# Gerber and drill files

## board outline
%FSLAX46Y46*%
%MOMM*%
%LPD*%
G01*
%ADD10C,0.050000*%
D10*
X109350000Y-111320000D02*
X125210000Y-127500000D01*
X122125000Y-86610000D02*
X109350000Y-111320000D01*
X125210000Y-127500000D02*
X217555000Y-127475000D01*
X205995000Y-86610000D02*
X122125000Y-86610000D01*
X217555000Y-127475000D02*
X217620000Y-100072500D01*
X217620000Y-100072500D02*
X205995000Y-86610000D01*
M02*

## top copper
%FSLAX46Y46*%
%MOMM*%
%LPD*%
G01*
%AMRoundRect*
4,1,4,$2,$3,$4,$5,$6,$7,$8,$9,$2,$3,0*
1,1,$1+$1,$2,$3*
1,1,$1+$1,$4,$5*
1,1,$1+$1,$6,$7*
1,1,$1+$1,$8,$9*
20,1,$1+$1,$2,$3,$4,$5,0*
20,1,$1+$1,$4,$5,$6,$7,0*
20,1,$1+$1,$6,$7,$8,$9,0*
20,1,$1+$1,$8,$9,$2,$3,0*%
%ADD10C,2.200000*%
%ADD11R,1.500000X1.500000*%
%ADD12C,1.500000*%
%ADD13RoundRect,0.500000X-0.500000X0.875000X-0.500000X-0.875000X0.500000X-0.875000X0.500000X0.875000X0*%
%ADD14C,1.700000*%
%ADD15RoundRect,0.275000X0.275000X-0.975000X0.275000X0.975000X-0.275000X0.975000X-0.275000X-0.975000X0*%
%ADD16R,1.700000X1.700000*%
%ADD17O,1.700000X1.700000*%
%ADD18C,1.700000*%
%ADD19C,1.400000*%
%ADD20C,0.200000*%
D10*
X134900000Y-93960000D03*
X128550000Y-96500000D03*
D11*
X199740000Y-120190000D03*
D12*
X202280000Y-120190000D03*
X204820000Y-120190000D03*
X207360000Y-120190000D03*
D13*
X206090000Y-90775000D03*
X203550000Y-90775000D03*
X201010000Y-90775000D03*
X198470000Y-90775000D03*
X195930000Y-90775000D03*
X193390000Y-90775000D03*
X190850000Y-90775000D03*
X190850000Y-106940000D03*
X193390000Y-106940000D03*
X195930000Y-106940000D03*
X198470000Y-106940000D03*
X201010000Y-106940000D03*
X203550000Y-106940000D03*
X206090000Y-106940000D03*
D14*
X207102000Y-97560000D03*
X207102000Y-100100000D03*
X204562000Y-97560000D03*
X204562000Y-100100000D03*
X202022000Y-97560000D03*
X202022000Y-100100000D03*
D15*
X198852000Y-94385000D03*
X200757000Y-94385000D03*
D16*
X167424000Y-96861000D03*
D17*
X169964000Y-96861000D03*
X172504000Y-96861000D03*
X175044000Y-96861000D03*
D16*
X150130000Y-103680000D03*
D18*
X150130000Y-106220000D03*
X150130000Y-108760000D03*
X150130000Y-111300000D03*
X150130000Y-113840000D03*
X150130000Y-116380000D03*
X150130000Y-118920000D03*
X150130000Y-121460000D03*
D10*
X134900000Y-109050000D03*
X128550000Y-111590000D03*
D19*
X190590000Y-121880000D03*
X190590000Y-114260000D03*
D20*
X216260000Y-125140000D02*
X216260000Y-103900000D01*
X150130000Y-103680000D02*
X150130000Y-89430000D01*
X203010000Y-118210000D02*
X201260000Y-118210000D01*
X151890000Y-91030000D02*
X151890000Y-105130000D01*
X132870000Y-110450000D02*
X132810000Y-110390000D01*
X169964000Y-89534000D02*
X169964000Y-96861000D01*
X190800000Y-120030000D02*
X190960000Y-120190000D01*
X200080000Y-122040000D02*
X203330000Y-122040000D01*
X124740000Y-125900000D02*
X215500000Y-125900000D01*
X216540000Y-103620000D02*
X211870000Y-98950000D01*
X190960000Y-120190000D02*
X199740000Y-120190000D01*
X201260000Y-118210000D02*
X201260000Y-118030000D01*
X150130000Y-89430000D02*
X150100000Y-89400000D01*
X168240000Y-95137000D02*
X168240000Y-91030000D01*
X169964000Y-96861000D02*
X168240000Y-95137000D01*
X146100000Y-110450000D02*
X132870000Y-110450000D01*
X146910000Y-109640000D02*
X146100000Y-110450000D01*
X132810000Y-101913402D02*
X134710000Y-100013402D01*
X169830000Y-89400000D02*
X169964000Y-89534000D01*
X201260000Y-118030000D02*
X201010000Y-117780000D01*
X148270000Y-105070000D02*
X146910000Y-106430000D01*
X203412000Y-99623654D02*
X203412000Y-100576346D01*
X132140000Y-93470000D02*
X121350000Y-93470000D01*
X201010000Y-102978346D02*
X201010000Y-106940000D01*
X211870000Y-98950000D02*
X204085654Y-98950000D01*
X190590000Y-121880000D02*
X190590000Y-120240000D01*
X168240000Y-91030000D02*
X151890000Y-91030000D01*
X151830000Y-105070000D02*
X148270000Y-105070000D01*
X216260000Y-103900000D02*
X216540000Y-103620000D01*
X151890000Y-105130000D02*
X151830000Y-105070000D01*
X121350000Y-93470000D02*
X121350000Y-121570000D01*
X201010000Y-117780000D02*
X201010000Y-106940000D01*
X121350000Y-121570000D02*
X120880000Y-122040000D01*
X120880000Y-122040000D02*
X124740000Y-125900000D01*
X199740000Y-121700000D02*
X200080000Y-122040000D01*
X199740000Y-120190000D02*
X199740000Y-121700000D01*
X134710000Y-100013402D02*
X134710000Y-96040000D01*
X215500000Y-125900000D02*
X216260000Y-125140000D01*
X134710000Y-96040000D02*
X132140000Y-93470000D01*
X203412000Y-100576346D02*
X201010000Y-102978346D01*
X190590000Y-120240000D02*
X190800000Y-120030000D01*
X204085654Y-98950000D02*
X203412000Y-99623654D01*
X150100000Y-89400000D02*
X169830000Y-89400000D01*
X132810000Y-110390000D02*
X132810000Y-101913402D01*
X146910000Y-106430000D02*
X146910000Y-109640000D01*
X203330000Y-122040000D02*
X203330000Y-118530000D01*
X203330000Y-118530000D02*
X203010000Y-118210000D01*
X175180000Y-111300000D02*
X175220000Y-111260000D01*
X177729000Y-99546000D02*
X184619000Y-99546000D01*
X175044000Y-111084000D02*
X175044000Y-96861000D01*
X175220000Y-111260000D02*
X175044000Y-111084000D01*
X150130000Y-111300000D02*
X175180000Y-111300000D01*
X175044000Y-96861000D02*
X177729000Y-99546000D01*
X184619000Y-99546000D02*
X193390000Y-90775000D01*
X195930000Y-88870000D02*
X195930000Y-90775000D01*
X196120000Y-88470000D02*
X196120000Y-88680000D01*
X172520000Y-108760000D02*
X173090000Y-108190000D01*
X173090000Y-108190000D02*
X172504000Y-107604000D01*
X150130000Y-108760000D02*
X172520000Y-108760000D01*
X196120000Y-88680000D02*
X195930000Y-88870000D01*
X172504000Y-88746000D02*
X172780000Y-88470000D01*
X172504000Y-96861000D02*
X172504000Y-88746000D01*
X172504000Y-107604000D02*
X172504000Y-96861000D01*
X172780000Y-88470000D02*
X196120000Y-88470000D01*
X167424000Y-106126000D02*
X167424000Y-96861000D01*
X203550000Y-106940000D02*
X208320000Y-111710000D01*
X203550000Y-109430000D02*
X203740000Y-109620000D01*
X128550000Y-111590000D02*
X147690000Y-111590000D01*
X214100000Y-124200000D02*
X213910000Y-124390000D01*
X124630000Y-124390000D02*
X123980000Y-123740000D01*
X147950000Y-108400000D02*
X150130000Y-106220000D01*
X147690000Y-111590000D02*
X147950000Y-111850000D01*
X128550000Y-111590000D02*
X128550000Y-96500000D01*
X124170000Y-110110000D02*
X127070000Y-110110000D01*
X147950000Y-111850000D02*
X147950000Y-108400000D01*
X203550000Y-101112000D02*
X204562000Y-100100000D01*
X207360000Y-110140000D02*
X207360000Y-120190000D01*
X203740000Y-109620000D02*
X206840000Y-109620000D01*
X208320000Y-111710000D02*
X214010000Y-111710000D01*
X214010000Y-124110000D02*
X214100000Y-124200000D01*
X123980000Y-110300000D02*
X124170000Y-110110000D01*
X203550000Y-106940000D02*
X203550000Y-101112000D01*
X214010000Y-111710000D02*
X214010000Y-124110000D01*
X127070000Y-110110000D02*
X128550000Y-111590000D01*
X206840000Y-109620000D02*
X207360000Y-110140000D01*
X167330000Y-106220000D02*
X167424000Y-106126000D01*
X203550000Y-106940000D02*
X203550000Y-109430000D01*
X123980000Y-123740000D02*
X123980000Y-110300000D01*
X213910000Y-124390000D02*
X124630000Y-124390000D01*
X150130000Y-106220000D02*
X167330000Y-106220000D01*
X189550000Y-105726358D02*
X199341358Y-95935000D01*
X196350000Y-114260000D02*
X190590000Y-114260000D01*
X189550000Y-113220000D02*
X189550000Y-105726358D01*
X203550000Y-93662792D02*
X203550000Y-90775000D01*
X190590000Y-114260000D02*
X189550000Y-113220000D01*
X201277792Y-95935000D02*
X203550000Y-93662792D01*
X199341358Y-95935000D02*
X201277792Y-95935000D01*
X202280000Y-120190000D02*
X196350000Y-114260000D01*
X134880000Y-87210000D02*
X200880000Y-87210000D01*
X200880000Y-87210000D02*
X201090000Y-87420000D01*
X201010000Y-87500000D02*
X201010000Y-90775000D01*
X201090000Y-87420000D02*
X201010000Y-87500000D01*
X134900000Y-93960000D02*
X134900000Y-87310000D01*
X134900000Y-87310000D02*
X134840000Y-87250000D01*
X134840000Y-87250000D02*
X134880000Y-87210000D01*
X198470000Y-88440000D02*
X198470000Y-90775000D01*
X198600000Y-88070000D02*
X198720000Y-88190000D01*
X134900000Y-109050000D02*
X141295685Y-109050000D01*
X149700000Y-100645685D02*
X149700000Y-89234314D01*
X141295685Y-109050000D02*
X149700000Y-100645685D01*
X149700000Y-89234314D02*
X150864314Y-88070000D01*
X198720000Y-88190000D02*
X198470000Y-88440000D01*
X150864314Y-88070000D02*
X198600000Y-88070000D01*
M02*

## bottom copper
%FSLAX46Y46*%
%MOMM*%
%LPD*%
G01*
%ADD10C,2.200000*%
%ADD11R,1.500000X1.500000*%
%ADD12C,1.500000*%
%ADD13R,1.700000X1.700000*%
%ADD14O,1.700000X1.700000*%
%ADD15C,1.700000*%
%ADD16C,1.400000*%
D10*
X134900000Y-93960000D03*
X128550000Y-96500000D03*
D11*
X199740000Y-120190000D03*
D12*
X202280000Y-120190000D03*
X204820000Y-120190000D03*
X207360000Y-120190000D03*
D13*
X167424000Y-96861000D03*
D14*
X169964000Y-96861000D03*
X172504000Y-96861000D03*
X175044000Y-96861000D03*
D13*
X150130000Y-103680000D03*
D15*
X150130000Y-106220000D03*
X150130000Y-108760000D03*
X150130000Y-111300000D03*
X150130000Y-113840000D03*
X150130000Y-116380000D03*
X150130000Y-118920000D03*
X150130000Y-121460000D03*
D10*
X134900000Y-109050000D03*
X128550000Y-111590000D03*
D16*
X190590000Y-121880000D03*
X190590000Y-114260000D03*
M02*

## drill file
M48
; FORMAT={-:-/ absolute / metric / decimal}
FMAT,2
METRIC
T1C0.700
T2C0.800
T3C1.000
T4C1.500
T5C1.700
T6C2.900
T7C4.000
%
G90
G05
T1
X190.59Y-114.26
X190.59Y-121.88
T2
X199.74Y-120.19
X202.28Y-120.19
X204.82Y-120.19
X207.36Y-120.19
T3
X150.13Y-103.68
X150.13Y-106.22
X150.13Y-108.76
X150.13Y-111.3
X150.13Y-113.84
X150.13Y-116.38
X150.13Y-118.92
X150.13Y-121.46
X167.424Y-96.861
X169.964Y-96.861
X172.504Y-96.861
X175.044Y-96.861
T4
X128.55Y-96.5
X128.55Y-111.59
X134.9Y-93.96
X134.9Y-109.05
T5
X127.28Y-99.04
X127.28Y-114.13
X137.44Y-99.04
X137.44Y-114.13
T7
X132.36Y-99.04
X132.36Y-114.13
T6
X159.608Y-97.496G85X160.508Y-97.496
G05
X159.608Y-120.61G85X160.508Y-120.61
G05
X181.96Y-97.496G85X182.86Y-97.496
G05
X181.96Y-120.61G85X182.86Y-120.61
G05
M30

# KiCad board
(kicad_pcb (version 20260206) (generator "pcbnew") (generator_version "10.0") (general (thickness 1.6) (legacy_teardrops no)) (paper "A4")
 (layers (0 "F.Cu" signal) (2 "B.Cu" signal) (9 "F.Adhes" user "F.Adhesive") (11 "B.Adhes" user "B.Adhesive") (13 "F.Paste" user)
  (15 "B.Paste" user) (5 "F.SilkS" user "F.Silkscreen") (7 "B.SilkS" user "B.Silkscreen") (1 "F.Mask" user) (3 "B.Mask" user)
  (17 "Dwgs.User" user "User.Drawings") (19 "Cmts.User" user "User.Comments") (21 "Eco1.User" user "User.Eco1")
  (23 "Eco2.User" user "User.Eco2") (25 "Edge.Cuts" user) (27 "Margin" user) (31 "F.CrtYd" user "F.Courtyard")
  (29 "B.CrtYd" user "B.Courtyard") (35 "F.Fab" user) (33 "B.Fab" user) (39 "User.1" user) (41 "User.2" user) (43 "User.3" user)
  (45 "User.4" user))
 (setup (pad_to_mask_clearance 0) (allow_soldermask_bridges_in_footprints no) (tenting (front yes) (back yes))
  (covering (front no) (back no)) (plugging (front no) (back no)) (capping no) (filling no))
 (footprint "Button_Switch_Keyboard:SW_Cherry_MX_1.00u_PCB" (layer "F.Cu") (at 134.9 93.96)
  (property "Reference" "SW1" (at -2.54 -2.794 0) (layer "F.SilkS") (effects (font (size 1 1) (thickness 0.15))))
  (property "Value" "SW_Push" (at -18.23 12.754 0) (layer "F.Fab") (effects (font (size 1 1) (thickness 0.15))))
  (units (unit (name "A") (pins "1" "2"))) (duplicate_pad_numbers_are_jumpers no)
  (pad "" np_thru_hole circle (at -7.62 5.08) (size 1.7 1.7) (drill 1.7) (layers "*.Cu" "*.Mask"))
  (pad "" np_thru_hole circle (at -2.54 5.08) (size 4 4) (drill 4) (layers "*.Cu" "*.Mask"))
  (pad "" np_thru_hole circle (at 2.54 5.08) (size 1.7 1.7) (drill 1.7) (layers "*.Cu" "*.Mask"))
  (pad "1" thru_hole circle (at 0 0) (size 2.2 2.2) (drill 1.5) (layers "*.Cu" "*.Mask") (remove_unused_layers no) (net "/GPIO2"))
  (pad "2" thru_hole circle (at -6.35 2.54) (size 2.2 2.2) (drill 1.5) (layers "*.Cu" "*.Mask") (remove_unused_layers no) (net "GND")))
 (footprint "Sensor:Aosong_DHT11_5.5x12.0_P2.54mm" (layer "F.Cu") (at 199.74 120.19 90)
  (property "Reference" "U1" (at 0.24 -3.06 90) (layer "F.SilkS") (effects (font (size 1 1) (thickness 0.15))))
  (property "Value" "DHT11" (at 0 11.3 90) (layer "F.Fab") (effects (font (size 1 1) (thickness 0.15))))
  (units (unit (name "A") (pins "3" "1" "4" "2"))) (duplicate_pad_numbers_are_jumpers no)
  (pad "1" thru_hole rect (at 0 0 90) (size 1.5 1.5) (drill 0.8) (layers "*.Cu" "*.Mask") (remove_unused_layers no) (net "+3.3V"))
  (pad "2" thru_hole circle (at 0 2.54 90) (size 1.5 1.5) (drill 0.8) (layers "*.Cu" "*.Mask") (remove_unused_layers no) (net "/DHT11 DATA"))
  (pad "3" thru_hole circle (at 0 5.08 90) (size 1.5 1.5) (drill 0.8) (layers "*.Cu" "*.Mask") (remove_unused_layers no)
   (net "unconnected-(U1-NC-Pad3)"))
  (pad "4" thru_hole circle (at 0 7.62 90) (size 1.5 1.5) (drill 0.8) (layers "*.Cu" "*.Mask") (remove_unused_layers no) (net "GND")))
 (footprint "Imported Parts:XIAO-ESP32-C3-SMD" (layer "F.Cu") (at 187.97 89.94 -90)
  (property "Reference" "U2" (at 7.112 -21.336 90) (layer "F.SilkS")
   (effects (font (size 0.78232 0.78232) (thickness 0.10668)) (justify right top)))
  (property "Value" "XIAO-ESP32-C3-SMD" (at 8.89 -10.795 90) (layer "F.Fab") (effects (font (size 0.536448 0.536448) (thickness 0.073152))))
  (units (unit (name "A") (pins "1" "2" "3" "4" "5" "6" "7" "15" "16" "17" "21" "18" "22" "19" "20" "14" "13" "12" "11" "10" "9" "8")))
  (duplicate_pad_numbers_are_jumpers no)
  (pad "1" smd roundrect (at 0.835 -18.12 270) (size 2.75 2) (layers "F.Cu" "F.Mask" "F.Paste") (roundrect_rratio 0.25)
   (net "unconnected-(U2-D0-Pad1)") (solder_mask_margin 0.0508) (thermal_bridge_angle 45))
  (pad "2" smd roundrect (at 0.835 -15.58 270) (size 2.75 2) (layers "F.Cu" "F.Mask" "F.Paste") (roundrect_rratio 0.25) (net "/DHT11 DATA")
   (solder_mask_margin 0.0508) (thermal_bridge_angle 45))
  (pad "3" smd roundrect (at 0.835 -13.04 270) (size 2.75 2) (layers "F.Cu" "F.Mask" "F.Paste") (roundrect_rratio 0.25) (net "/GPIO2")
   (solder_mask_margin 0.0508) (thermal_bridge_angle 45))
  (pad "4" smd roundrect (at 0.835 -10.5 270) (size 2.75 2) (layers "F.Cu" "F.Mask" "F.Paste") (roundrect_rratio 0.25) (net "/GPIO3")
   (solder_mask_margin 0.0508) (thermal_bridge_angle 45))
  (pad "5" smd roundrect (at 0.835 -7.96 270) (size 2.75 2) (layers "F.Cu" "F.Mask" "F.Paste") (roundrect_rratio 0.25) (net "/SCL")
   (solder_mask_margin 0.0508) (thermal_bridge_angle 45))
  (pad "6" smd roundrect (at 0.835 -5.42 270) (size 2.75 2) (layers "F.Cu" "F.Mask" "F.Paste") (roundrect_rratio 0.25) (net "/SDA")
   (solder_mask_margin 0.0508) (thermal_bridge_angle 45))
  (pad "7" smd roundrect (at 0.835 -2.88 270) (size 2.75 2) (layers "F.Cu" "F.Mask" "F.Paste") (roundrect_rratio 0.25)
   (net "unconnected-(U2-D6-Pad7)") (solder_mask_margin 0.0508) (thermal_bridge_angle 45))
  (pad "8" smd roundrect (at 17 -2.88 270) (size 2.75 2) (layers "F.Cu" "F.Mask" "F.Paste") (roundrect_rratio 0.25)
   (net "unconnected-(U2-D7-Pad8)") (solder_mask_margin 0.0508) (thermal_bridge_angle 45))
  (pad "9" smd roundrect (at 17 -5.42 270) (size 2.75 2) (layers "F.Cu" "F.Mask" "F.Paste") (roundrect_rratio 0.25)
   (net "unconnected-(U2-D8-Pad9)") (solder_mask_margin 0.0508) (thermal_bridge_angle 45))
  (pad "10" smd roundrect (at 17 -7.96 270) (size 2.75 2) (layers "F.Cu" "F.Mask" "F.Paste") (roundrect_rratio 0.25)
   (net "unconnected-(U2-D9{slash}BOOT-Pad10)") (solder_mask_margin 0.0508) (thermal_bridge_angle 45))
  (pad "11" smd roundrect (at 17 -10.5 270) (size 2.75 2) (layers "F.Cu" "F.Mask" "F.Paste") (roundrect_rratio 0.25)
   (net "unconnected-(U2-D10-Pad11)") (solder_mask_margin 0.0508) (thermal_bridge_angle 45))
  (pad "12" smd roundrect (at 17 -13.04 270) (size 2.75 2) (layers "F.Cu" "F.Mask" "F.Paste") (roundrect_rratio 0.25) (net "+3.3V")
   (solder_mask_margin 0.0508) (thermal_bridge_angle 45))
  (pad "13" smd roundrect (at 17 -15.58 270) (size 2.75 2) (layers "F.Cu" "F.Mask" "F.Paste") (roundrect_rratio 0.25) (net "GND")
   (solder_mask_margin 0.0508) (thermal_bridge_angle 45))
  (pad "14" smd roundrect (at 17 -18.12 270) (size 2.75 2) (layers "F.Cu" "F.Mask" "F.Paste") (roundrect_rratio 0.25) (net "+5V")
   (solder_mask_margin 0.0508) (thermal_bridge_angle 45))
  (pad "15" smd circle (at 7.62 -19.132 270) (size 1.7 1.7) (layers "F.Cu" "F.Mask" "F.Paste") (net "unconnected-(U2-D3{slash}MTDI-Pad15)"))
  (pad "16" smd circle (at 10.16 -19.132 270) (size 1.7 1.7) (layers "F.Cu" "F.Mask" "F.Paste") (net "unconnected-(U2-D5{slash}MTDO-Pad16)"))
  (pad "17" smd circle (at 7.62 -16.592 270) (size 1.7 1.7) (layers "F.Cu" "F.Mask" "F.Paste") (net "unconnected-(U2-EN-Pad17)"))
  (pad "18" smd circle (at 10.16 -16.592 270) (size 1.7 1.7) (layers "F.Cu" "F.Mask" "F.Paste") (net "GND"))
  (pad "19" smd circle (at 7.62 -14.052 270) (size 1.7 1.7) (layers "F.Cu" "F.Mask" "F.Paste") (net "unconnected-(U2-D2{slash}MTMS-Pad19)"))
  (pad "20" smd circle (at 10.16 -14.052 270) (size 1.7 1.7) (layers "F.Cu" "F.Mask" "F.Paste") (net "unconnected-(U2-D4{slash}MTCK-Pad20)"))
  (pad "21" smd roundrect (at 4.445 -10.882 90) (size 2.5 1.1) (layers "F.Cu" "F.Mask" "F.Paste") (roundrect_rratio 0.25)
   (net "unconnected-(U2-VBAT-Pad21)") (thermal_bridge_angle 45))
  (pad "22" smd roundrect (at 4.445 -12.787 90) (size 2.5 1.1) (layers "F.Cu" "F.Mask" "F.Paste") (roundrect_rratio 0.25)
   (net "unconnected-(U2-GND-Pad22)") (thermal_bridge_angle 45)))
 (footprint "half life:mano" (layer "F.Cu") (at 180.8 111.37)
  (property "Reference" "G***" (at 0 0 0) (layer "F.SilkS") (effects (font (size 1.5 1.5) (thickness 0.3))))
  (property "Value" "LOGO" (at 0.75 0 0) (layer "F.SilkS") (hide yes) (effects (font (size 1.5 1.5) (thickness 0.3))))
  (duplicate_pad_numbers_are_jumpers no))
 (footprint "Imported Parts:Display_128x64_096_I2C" (layer "F.Cu") (at 171.234 96.861)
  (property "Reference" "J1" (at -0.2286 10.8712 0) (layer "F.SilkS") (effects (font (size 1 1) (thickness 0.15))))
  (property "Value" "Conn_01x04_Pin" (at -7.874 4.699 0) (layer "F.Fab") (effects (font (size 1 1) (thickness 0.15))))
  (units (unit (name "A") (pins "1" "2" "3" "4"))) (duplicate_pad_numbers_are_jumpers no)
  (pad "" np_thru_hole oval (at -11.176 0.635) (size 3.8 2.9) (drill oval 3.8 2.9) (layers "*.Cu" "*.Mask"))
  (pad "" np_thru_hole oval (at -11.176 23.749) (size 3.8 2.9) (drill oval 3.8 2.9) (layers "*.Cu" "*.Mask"))
  (pad "" np_thru_hole oval (at 11.176 0.635) (size 3.8 2.9) (drill oval 3.8 2.9) (layers "*.Cu" "*.Mask"))
  (pad "" np_thru_hole oval (at 11.176 23.749) (size 3.8 2.9) (drill oval 3.8 2.9) (layers "*.Cu" "*.Mask"))
  (pad "1" thru_hole rect (at -3.81 0 90) (size 1.7 1.7) (drill 1) (layers "*.Cu" "*.Mask") (remove_unused_layers no) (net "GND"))
  (pad "2" thru_hole oval (at -1.27 0 90) (size 1.7 1.7) (drill 1) (layers "*.Cu" "*.Mask") (remove_unused_layers no) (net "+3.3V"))
  (pad "3" thru_hole oval (at 1.27 0 90) (size 1.7 1.7) (drill 1) (layers "*.Cu" "*.Mask") (remove_unused_layers no) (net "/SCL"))
  (pad "4" thru_hole oval (at 3.81 0 90) (size 1.7 1.7) (drill 1) (layers "*.Cu" "*.Mask") (remove_unused_layers no) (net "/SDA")))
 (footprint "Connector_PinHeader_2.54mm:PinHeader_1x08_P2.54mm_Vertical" (layer "F.Cu") (at 150.13 103.68)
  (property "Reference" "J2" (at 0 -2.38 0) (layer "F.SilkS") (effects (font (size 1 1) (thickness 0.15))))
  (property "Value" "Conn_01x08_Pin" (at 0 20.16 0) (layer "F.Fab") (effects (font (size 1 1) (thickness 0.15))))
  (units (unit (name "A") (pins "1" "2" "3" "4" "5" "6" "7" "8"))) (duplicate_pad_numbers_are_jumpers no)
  (pad "1" thru_hole rect (at 0 0) (size 1.7 1.7) (drill 1) (layers "*.Cu" "*.Mask") (remove_unused_layers no) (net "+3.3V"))
  (pad "2" thru_hole circle (at 0 2.54) (size 1.7 1.7) (drill 1) (layers "*.Cu" "*.Mask") (remove_unused_layers no) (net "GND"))
  (pad "3" thru_hole circle (at 0 5.08) (size 1.7 1.7) (drill 1) (layers "*.Cu" "*.Mask") (remove_unused_layers no) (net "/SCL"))
  (pad "4" thru_hole circle (at 0 7.62) (size 1.7 1.7) (drill 1) (layers "*.Cu" "*.Mask") (remove_unused_layers no) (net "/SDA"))
  (pad "5" thru_hole circle (at 0 10.16) (size 1.7 1.7) (drill 1) (layers "*.Cu" "*.Mask") (remove_unused_layers no)
   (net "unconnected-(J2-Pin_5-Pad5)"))
  (pad "6" thru_hole circle (at 0 12.7) (size 1.7 1.7) (drill 1) (layers "*.Cu" "*.Mask") (remove_unused_layers no)
   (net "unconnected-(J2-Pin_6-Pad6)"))
  (pad "7" thru_hole circle (at 0 15.24) (size 1.7 1.7) (drill 1) (layers "*.Cu" "*.Mask") (remove_unused_layers no)
   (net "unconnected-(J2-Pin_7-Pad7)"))
  (pad "8" thru_hole circle (at 0 17.78) (size 1.7 1.7) (drill 1) (layers "*.Cu" "*.Mask") (remove_unused_layers no)
   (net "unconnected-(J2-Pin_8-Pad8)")))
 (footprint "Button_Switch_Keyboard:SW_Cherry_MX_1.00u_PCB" (layer "F.Cu") (at 134.9 109.05)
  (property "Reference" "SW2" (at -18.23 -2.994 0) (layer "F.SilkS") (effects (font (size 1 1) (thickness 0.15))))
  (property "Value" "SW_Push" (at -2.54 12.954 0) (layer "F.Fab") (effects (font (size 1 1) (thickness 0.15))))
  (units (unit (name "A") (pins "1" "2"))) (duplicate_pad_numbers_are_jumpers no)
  (pad "" np_thru_hole circle (at -7.62 5.08) (size 1.7 1.7) (drill 1.7) (layers "*.Cu" "*.Mask"))
  (pad "" np_thru_hole circle (at -2.54 5.08) (size 4 4) (drill 4) (layers "*.Cu" "*.Mask"))
  (pad "" np_thru_hole circle (at 2.54 5.08) (size 1.7 1.7) (drill 1.7) (layers "*.Cu" "*.Mask"))
  (pad "1" thru_hole circle (at 0 0) (size 2.2 2.2) (drill 1.5) (layers "*.Cu" "*.Mask") (remove_unused_layers no) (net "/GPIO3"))
  (pad "2" thru_hole circle (at -6.35 2.54) (size 2.2 2.2) (drill 1.5) (layers "*.Cu" "*.Mask") (remove_unused_layers no) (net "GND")))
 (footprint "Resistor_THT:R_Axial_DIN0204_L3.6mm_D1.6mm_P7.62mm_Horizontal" (layer "F.Cu") (at 190.59 121.88 90)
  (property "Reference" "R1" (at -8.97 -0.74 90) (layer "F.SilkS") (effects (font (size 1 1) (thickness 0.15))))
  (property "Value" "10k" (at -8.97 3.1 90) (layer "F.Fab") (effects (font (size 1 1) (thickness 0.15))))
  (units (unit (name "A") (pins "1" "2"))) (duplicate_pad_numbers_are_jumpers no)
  (pad "1" thru_hole circle (at 0 0 90) (size 1.4 1.4) (drill 0.7) (layers "*.Cu" "*.Mask") (remove_unused_layers no) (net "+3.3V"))
  (pad "2" thru_hole circle (at 7.62 0 90) (size 1.4 1.4) (drill 0.7) (layers "*.Cu" "*.Mask") (remove_unused_layers no) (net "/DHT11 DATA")))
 (gr_line (start 109.35 111.32) (end 125.21 127.5) (stroke (width 0.05) (type default)) (layer "Edge.Cuts"))
 (gr_line (start 122.125 86.61) (end 109.35 111.32) (stroke (width 0.05) (type default)) (layer "Edge.Cuts"))
 (gr_line (start 125.21 127.5) (end 217.555 127.475) (stroke (width 0.05) (type solid)) (layer "Edge.Cuts"))
 (gr_line (start 205.995 86.61) (end 122.125 86.61) (stroke (width 0.05) (type solid)) (layer "Edge.Cuts"))
 (gr_line (start 217.555 127.475) (end 217.62 100.0725) (stroke (width 0.05) (type solid)) (layer "Edge.Cuts"))
 (gr_line (start 217.62 100.0725) (end 205.995 86.61) (stroke (width 0.05) (type default)) (layer "Edge.Cuts"))
 (segment (start 216.26 125.14) (end 216.26 103.9) (width 0.2) (layer "F.Cu") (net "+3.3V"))
 (segment (start 150.13 103.68) (end 150.13 89.43) (width 0.2) (layer "F.Cu") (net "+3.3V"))
 (segment (start 203.01 118.21) (end 201.26 118.21) (width 0.2) (layer "F.Cu") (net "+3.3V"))
 (segment (start 151.89 91.03) (end 151.89 105.13) (width 0.2) (layer "F.Cu") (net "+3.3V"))
 (segment (start 132.87 110.45) (end 132.81 110.39) (width 0.2) (layer "F.Cu") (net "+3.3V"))
 (segment (start 169.964 89.534) (end 169.964 96.861) (width 0.2) (layer "F.Cu") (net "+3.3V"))
 (segment (start 190.8 120.03) (end 190.96 120.19) (width 0.2) (layer "F.Cu") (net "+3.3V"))
 (segment (start 200.08 122.04) (end 203.33 122.04) (width 0.2) (layer "F.Cu") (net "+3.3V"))
 (segment (start 124.74 125.9) (end 215.5 125.9) (width 0.2) (layer "F.Cu") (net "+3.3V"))
 (segment (start 216.54 103.62) (end 211.87 98.95) (width 0.2) (layer "F.Cu") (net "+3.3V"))
 (segment (start 190.96 120.19) (end 199.74 120.19) (width 0.2) (layer "F.Cu") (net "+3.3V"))
 (segment (start 201.26 118.21) (end 201.26 118.03) (width 0.2) (layer "F.Cu") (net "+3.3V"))
 (segment (start 150.13 89.43) (end 150.1 89.4) (width 0.2) (layer "F.Cu") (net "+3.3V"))
 (segment (start 168.24 95.137) (end 168.24 91.03) (width 0.2) (layer "F.Cu") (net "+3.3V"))
 (segment (start 169.964 96.861) (end 168.24 95.137) (width 0.2) (layer "F.Cu") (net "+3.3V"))
 (segment (start 146.1 110.45) (end 132.87 110.45) (width 0.2) (layer "F.Cu") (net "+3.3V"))
 (segment (start 146.91 109.64) (end 146.1 110.45) (width 0.2) (layer "F.Cu") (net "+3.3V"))
 (segment (start 132.81 101.913402) (end 134.71 100.013402) (width 0.2) (layer "F.Cu") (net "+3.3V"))
 (segment (start 169.83 89.4) (end 169.964 89.534) (width 0.2) (layer "F.Cu") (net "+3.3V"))
 (segment (start 201.26 118.03) (end 201.01 117.78) (width 0.2) (layer "F.Cu") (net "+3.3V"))
 (segment (start 148.27 105.07) (end 146.91 106.43) (width 0.2) (layer "F.Cu") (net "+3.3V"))
 (segment (start 203.412 99.623654) (end 203.412 100.576346) (width 0.2) (layer "F.Cu") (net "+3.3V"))
 (segment (start 132.14 93.47) (end 121.35 93.47) (width 0.2) (layer "F.Cu") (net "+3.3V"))
 (segment (start 201.01 102.978346) (end 201.01 106.94) (width 0.2) (layer "F.Cu") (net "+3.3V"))
 (segment (start 211.87 98.95) (end 204.085654 98.95) (width 0.2) (layer "F.Cu") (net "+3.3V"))
 (segment (start 190.59 121.88) (end 190.59 120.24) (width 0.2) (layer "F.Cu") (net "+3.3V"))
 (segment (start 168.24 91.03) (end 151.89 91.03) (width 0.2) (layer "F.Cu") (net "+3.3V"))
 (segment (start 151.83 105.07) (end 148.27 105.07) (width 0.2) (layer "F.Cu") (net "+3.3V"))
 (segment (start 216.26 103.9) (end 216.54 103.62) (width 0.2) (layer "F.Cu") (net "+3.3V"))
 (segment (start 151.89 105.13) (end 151.83 105.07) (width 0.2) (layer "F.Cu") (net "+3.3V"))
 (segment (start 121.35 93.47) (end 121.35 121.57) (width 0.2) (layer "F.Cu") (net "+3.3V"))
 (segment (start 201.01 117.78) (end 201.01 106.94) (width 0.2) (layer "F.Cu") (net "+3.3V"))
 (segment (start 121.35 121.57) (end 120.88 122.04) (width 0.2) (layer "F.Cu") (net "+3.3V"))
 (segment (start 120.88 122.04) (end 124.74 125.9) (width 0.2) (layer "F.Cu") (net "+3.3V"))
 (segment (start 199.74 121.7) (end 200.08 122.04) (width 0.2) (layer "F.Cu") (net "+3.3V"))
 (segment (start 199.74 120.19) (end 199.74 121.7) (width 0.2) (layer "F.Cu") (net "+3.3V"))
 (segment (start 134.71 100.013402) (end 134.71 96.04) (width 0.2) (layer "F.Cu") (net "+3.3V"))
 (segment (start 215.5 125.9) (end 216.26 125.14) (width 0.2) (layer "F.Cu") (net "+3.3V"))
 (segment (start 134.71 96.04) (end 132.14 93.47) (width 0.2) (layer "F.Cu") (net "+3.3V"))
 (segment (start 203.412 100.576346) (end 201.01 102.978346) (width 0.2) (layer "F.Cu") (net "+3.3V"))
 (segment (start 190.59 120.24) (end 190.8 120.03) (width 0.2) (layer "F.Cu") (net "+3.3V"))
 (segment (start 204.085654 98.95) (end 203.412 99.623654) (width 0.2) (layer "F.Cu") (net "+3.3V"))
 (segment (start 150.1 89.4) (end 169.83 89.4) (width 0.2) (layer "F.Cu") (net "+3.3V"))
 (segment (start 132.81 110.39) (end 132.81 101.913402) (width 0.2) (layer "F.Cu") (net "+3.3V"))
 (segment (start 146.91 106.43) (end 146.91 109.64) (width 0.2) (layer "F.Cu") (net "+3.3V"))
 (segment (start 203.33 122.04) (end 203.33 118.53) (width 0.2) (layer "F.Cu") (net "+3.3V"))
 (segment (start 203.33 118.53) (end 203.01 118.21) (width 0.2) (layer "F.Cu") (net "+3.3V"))
 (segment (start 175.18 111.3) (end 175.22 111.26) (width 0.2) (layer "F.Cu") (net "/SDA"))
 (segment (start 177.729 99.546) (end 184.619 99.546) (width 0.2) (layer "F.Cu") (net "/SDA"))
 (segment (start 175.044 111.084) (end 175.044 96.861) (width 0.2) (layer "F.Cu") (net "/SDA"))
 (segment (start 175.22 111.26) (end 175.044 111.084) (width 0.2) (layer "F.Cu") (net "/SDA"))
 (segment (start 150.13 111.3) (end 175.18 111.3) (width 0.2) (layer "F.Cu") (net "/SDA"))
 (segment (start 175.044 96.861) (end 177.729 99.546) (width 0.2) (layer "F.Cu") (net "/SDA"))
 (segment (start 184.619 99.546) (end 193.39 90.775) (width 0.2) (layer "F.Cu") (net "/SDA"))
 (segment (start 195.93 88.87) (end 195.93 90.775) (width 0.2) (layer "F.Cu") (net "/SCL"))
 (segment (start 196.12 88.47) (end 196.12 88.68) (width 0.2) (layer "F.Cu") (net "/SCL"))
 (segment (start 172.52 108.76) (end 173.09 108.19) (width 0.2) (layer "F.Cu") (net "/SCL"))
 (segment (start 173.09 108.19) (end 172.504 107.604) (width 0.2) (layer "F.Cu") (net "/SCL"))
 (segment (start 150.13 108.76) (end 172.52 108.76) (width 0.2) (layer "F.Cu") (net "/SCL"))
 (segment (start 196.12 88.68) (end 195.93 88.87) (width 0.2) (layer "F.Cu") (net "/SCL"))
 (segment (start 172.504 88.746) (end 172.78 88.47) (width 0.2) (layer "F.Cu") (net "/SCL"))
 (segment (start 172.504 96.861) (end 172.504 88.746) (width 0.2) (layer "F.Cu") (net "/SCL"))
 (segment (start 172.504 107.604) (end 172.504 96.861) (width 0.2) (layer "F.Cu") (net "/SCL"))
 (segment (start 172.78 88.47) (end 196.12 88.47) (width 0.2) (layer "F.Cu") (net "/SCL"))
 (segment (start 167.424 106.126) (end 167.424 96.861) (width 0.2) (layer "F.Cu") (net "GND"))
 (segment (start 203.55 106.94) (end 208.32 111.71) (width 0.2) (layer "F.Cu") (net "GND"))
 (segment (start 203.55 109.43) (end 203.74 109.62) (width 0.2) (layer "F.Cu") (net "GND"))
 (segment (start 128.55 111.59) (end 147.69 111.59) (width 0.2) (layer "F.Cu") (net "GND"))
 (segment (start 214.1 124.2) (end 213.91 124.39) (width 0.2) (layer "F.Cu") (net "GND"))
 (segment (start 124.63 124.39) (end 123.98 123.74) (width 0.2) (layer "F.Cu") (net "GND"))
 (segment (start 147.95 108.4) (end 150.13 106.22) (width 0.2) (layer "F.Cu") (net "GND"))
 (segment (start 147.69 111.59) (end 147.95 111.85) (width 0.2) (layer "F.Cu") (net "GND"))
 (segment (start 128.55 111.59) (end 128.55 96.5) (width 0.2) (layer "F.Cu") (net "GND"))
 (segment (start 124.17 110.11) (end 127.07 110.11) (width 0.2) (layer "F.Cu") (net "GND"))
 (segment (start 147.95 111.85) (end 147.95 108.4) (width 0.2) (layer "F.Cu") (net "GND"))
 (segment (start 203.55 101.112) (end 204.562 100.1) (width 0.2) (layer "F.Cu") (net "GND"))
 (segment (start 207.36 110.14) (end 207.36 120.19) (width 0.2) (layer "F.Cu") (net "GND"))
 (segment (start 203.74 109.62) (end 206.84 109.62) (width 0.2) (layer "F.Cu") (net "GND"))
 (segment (start 208.32 111.71) (end 214.01 111.71) (width 0.2) (layer "F.Cu") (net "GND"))
 (segment (start 214.01 124.11) (end 214.1 124.2) (width 0.2) (layer "F.Cu") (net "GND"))
 (segment (start 123.98 110.3) (end 124.17 110.11) (width 0.2) (layer "F.Cu") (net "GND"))
 (segment (start 203.55 106.94) (end 203.55 101.112) (width 0.2) (layer "F.Cu") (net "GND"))
 (segment (start 214.01 111.71) (end 214.01 124.11) (width 0.2) (layer "F.Cu") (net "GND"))
 (segment (start 127.07 110.11) (end 128.55 111.59) (width 0.2) (layer "F.Cu") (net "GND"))
 (segment (start 206.84 109.62) (end 207.36 110.14) (width 0.2) (layer "F.Cu") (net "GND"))
 (segment (start 167.33 106.22) (end 167.424 106.126) (width 0.2) (layer "F.Cu") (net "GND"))
 (segment (start 203.55 106.94) (end 203.55 109.43) (width 0.2) (layer "F.Cu") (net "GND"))
 (segment (start 123.98 123.74) (end 123.98 110.3) (width 0.2) (layer "F.Cu") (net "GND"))
 (segment (start 213.91 124.39) (end 124.63 124.39) (width 0.2) (layer "F.Cu") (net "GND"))
 (segment (start 150.13 106.22) (end 167.33 106.22) (width 0.2) (layer "F.Cu") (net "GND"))
 (segment (start 189.55 105.726358) (end 199.341358 95.935) (width 0.2) (layer "F.Cu") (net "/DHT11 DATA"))
 (segment (start 196.35 114.26) (end 190.59 114.26) (width 0.2) (layer "F.Cu") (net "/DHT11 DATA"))
 (segment (start 189.55 113.22) (end 189.55 105.726358) (width 0.2) (layer "F.Cu") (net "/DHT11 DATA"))
 (segment (start 203.55 93.662792) (end 203.55 90.775) (width 0.2) (layer "F.Cu") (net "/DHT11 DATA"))
 (segment (start 190.59 114.26) (end 189.55 113.22) (width 0.2) (layer "F.Cu") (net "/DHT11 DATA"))
 (segment (start 201.277792 95.935) (end 203.55 93.662792) (width 0.2) (layer "F.Cu") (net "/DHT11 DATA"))
 (segment (start 199.341358 95.935) (end 201.277792 95.935) (width 0.2) (layer "F.Cu") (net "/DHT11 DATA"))
 (segment (start 202.28 120.19) (end 196.35 114.26) (width 0.2) (layer "F.Cu") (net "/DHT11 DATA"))
 (segment (start 134.88 87.21) (end 200.88 87.21) (width 0.2) (layer "F.Cu") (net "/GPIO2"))
 (segment (start 200.88 87.21) (end 201.09 87.42) (width 0.2) (layer "F.Cu") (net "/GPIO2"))
 (segment (start 201.01 87.5) (end 201.01 90.775) (width 0.2) (layer "F.Cu") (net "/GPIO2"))
 (segment (start 201.09 87.42) (end 201.01 87.5) (width 0.2) (layer "F.Cu") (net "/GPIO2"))
 (segment (start 134.9 93.96) (end 134.9 87.31) (width 0.2) (layer "F.Cu") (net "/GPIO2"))
 (segment (start 134.9 87.31) (end 134.84 87.25) (width 0.2) (layer "F.Cu") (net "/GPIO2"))
 (segment (start 134.84 87.25) (end 134.88 87.21) (width 0.2) (layer "F.Cu") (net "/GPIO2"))
 (segment (start 198.47 88.44) (end 198.47 90.775) (width 0.2) (layer "F.Cu") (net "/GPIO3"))
 (segment (start 198.6 88.07) (end 198.72 88.19) (width 0.2) (layer "F.Cu") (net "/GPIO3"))
 (segment (start 134.9 109.05) (end 141.295685 109.05) (width 0.2) (layer "F.Cu") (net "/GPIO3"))
 (segment (start 149.7 100.645685) (end 149.7 89.234314) (width 0.2) (layer "F.Cu") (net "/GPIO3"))
 (segment (start 141.295685 109.05) (end 149.7 100.645685) (width 0.2) (layer "F.Cu") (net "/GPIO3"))
 (segment (start 149.7 89.234314) (end 150.864314 88.07) (width 0.2) (layer "F.Cu") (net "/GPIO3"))
 (segment (start 198.72 88.19) (end 198.47 88.44) (width 0.2) (layer "F.Cu") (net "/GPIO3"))
 (segment (start 150.864314 88.07) (end 198.6 88.07) (width 0.2) (layer "F.Cu") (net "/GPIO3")))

